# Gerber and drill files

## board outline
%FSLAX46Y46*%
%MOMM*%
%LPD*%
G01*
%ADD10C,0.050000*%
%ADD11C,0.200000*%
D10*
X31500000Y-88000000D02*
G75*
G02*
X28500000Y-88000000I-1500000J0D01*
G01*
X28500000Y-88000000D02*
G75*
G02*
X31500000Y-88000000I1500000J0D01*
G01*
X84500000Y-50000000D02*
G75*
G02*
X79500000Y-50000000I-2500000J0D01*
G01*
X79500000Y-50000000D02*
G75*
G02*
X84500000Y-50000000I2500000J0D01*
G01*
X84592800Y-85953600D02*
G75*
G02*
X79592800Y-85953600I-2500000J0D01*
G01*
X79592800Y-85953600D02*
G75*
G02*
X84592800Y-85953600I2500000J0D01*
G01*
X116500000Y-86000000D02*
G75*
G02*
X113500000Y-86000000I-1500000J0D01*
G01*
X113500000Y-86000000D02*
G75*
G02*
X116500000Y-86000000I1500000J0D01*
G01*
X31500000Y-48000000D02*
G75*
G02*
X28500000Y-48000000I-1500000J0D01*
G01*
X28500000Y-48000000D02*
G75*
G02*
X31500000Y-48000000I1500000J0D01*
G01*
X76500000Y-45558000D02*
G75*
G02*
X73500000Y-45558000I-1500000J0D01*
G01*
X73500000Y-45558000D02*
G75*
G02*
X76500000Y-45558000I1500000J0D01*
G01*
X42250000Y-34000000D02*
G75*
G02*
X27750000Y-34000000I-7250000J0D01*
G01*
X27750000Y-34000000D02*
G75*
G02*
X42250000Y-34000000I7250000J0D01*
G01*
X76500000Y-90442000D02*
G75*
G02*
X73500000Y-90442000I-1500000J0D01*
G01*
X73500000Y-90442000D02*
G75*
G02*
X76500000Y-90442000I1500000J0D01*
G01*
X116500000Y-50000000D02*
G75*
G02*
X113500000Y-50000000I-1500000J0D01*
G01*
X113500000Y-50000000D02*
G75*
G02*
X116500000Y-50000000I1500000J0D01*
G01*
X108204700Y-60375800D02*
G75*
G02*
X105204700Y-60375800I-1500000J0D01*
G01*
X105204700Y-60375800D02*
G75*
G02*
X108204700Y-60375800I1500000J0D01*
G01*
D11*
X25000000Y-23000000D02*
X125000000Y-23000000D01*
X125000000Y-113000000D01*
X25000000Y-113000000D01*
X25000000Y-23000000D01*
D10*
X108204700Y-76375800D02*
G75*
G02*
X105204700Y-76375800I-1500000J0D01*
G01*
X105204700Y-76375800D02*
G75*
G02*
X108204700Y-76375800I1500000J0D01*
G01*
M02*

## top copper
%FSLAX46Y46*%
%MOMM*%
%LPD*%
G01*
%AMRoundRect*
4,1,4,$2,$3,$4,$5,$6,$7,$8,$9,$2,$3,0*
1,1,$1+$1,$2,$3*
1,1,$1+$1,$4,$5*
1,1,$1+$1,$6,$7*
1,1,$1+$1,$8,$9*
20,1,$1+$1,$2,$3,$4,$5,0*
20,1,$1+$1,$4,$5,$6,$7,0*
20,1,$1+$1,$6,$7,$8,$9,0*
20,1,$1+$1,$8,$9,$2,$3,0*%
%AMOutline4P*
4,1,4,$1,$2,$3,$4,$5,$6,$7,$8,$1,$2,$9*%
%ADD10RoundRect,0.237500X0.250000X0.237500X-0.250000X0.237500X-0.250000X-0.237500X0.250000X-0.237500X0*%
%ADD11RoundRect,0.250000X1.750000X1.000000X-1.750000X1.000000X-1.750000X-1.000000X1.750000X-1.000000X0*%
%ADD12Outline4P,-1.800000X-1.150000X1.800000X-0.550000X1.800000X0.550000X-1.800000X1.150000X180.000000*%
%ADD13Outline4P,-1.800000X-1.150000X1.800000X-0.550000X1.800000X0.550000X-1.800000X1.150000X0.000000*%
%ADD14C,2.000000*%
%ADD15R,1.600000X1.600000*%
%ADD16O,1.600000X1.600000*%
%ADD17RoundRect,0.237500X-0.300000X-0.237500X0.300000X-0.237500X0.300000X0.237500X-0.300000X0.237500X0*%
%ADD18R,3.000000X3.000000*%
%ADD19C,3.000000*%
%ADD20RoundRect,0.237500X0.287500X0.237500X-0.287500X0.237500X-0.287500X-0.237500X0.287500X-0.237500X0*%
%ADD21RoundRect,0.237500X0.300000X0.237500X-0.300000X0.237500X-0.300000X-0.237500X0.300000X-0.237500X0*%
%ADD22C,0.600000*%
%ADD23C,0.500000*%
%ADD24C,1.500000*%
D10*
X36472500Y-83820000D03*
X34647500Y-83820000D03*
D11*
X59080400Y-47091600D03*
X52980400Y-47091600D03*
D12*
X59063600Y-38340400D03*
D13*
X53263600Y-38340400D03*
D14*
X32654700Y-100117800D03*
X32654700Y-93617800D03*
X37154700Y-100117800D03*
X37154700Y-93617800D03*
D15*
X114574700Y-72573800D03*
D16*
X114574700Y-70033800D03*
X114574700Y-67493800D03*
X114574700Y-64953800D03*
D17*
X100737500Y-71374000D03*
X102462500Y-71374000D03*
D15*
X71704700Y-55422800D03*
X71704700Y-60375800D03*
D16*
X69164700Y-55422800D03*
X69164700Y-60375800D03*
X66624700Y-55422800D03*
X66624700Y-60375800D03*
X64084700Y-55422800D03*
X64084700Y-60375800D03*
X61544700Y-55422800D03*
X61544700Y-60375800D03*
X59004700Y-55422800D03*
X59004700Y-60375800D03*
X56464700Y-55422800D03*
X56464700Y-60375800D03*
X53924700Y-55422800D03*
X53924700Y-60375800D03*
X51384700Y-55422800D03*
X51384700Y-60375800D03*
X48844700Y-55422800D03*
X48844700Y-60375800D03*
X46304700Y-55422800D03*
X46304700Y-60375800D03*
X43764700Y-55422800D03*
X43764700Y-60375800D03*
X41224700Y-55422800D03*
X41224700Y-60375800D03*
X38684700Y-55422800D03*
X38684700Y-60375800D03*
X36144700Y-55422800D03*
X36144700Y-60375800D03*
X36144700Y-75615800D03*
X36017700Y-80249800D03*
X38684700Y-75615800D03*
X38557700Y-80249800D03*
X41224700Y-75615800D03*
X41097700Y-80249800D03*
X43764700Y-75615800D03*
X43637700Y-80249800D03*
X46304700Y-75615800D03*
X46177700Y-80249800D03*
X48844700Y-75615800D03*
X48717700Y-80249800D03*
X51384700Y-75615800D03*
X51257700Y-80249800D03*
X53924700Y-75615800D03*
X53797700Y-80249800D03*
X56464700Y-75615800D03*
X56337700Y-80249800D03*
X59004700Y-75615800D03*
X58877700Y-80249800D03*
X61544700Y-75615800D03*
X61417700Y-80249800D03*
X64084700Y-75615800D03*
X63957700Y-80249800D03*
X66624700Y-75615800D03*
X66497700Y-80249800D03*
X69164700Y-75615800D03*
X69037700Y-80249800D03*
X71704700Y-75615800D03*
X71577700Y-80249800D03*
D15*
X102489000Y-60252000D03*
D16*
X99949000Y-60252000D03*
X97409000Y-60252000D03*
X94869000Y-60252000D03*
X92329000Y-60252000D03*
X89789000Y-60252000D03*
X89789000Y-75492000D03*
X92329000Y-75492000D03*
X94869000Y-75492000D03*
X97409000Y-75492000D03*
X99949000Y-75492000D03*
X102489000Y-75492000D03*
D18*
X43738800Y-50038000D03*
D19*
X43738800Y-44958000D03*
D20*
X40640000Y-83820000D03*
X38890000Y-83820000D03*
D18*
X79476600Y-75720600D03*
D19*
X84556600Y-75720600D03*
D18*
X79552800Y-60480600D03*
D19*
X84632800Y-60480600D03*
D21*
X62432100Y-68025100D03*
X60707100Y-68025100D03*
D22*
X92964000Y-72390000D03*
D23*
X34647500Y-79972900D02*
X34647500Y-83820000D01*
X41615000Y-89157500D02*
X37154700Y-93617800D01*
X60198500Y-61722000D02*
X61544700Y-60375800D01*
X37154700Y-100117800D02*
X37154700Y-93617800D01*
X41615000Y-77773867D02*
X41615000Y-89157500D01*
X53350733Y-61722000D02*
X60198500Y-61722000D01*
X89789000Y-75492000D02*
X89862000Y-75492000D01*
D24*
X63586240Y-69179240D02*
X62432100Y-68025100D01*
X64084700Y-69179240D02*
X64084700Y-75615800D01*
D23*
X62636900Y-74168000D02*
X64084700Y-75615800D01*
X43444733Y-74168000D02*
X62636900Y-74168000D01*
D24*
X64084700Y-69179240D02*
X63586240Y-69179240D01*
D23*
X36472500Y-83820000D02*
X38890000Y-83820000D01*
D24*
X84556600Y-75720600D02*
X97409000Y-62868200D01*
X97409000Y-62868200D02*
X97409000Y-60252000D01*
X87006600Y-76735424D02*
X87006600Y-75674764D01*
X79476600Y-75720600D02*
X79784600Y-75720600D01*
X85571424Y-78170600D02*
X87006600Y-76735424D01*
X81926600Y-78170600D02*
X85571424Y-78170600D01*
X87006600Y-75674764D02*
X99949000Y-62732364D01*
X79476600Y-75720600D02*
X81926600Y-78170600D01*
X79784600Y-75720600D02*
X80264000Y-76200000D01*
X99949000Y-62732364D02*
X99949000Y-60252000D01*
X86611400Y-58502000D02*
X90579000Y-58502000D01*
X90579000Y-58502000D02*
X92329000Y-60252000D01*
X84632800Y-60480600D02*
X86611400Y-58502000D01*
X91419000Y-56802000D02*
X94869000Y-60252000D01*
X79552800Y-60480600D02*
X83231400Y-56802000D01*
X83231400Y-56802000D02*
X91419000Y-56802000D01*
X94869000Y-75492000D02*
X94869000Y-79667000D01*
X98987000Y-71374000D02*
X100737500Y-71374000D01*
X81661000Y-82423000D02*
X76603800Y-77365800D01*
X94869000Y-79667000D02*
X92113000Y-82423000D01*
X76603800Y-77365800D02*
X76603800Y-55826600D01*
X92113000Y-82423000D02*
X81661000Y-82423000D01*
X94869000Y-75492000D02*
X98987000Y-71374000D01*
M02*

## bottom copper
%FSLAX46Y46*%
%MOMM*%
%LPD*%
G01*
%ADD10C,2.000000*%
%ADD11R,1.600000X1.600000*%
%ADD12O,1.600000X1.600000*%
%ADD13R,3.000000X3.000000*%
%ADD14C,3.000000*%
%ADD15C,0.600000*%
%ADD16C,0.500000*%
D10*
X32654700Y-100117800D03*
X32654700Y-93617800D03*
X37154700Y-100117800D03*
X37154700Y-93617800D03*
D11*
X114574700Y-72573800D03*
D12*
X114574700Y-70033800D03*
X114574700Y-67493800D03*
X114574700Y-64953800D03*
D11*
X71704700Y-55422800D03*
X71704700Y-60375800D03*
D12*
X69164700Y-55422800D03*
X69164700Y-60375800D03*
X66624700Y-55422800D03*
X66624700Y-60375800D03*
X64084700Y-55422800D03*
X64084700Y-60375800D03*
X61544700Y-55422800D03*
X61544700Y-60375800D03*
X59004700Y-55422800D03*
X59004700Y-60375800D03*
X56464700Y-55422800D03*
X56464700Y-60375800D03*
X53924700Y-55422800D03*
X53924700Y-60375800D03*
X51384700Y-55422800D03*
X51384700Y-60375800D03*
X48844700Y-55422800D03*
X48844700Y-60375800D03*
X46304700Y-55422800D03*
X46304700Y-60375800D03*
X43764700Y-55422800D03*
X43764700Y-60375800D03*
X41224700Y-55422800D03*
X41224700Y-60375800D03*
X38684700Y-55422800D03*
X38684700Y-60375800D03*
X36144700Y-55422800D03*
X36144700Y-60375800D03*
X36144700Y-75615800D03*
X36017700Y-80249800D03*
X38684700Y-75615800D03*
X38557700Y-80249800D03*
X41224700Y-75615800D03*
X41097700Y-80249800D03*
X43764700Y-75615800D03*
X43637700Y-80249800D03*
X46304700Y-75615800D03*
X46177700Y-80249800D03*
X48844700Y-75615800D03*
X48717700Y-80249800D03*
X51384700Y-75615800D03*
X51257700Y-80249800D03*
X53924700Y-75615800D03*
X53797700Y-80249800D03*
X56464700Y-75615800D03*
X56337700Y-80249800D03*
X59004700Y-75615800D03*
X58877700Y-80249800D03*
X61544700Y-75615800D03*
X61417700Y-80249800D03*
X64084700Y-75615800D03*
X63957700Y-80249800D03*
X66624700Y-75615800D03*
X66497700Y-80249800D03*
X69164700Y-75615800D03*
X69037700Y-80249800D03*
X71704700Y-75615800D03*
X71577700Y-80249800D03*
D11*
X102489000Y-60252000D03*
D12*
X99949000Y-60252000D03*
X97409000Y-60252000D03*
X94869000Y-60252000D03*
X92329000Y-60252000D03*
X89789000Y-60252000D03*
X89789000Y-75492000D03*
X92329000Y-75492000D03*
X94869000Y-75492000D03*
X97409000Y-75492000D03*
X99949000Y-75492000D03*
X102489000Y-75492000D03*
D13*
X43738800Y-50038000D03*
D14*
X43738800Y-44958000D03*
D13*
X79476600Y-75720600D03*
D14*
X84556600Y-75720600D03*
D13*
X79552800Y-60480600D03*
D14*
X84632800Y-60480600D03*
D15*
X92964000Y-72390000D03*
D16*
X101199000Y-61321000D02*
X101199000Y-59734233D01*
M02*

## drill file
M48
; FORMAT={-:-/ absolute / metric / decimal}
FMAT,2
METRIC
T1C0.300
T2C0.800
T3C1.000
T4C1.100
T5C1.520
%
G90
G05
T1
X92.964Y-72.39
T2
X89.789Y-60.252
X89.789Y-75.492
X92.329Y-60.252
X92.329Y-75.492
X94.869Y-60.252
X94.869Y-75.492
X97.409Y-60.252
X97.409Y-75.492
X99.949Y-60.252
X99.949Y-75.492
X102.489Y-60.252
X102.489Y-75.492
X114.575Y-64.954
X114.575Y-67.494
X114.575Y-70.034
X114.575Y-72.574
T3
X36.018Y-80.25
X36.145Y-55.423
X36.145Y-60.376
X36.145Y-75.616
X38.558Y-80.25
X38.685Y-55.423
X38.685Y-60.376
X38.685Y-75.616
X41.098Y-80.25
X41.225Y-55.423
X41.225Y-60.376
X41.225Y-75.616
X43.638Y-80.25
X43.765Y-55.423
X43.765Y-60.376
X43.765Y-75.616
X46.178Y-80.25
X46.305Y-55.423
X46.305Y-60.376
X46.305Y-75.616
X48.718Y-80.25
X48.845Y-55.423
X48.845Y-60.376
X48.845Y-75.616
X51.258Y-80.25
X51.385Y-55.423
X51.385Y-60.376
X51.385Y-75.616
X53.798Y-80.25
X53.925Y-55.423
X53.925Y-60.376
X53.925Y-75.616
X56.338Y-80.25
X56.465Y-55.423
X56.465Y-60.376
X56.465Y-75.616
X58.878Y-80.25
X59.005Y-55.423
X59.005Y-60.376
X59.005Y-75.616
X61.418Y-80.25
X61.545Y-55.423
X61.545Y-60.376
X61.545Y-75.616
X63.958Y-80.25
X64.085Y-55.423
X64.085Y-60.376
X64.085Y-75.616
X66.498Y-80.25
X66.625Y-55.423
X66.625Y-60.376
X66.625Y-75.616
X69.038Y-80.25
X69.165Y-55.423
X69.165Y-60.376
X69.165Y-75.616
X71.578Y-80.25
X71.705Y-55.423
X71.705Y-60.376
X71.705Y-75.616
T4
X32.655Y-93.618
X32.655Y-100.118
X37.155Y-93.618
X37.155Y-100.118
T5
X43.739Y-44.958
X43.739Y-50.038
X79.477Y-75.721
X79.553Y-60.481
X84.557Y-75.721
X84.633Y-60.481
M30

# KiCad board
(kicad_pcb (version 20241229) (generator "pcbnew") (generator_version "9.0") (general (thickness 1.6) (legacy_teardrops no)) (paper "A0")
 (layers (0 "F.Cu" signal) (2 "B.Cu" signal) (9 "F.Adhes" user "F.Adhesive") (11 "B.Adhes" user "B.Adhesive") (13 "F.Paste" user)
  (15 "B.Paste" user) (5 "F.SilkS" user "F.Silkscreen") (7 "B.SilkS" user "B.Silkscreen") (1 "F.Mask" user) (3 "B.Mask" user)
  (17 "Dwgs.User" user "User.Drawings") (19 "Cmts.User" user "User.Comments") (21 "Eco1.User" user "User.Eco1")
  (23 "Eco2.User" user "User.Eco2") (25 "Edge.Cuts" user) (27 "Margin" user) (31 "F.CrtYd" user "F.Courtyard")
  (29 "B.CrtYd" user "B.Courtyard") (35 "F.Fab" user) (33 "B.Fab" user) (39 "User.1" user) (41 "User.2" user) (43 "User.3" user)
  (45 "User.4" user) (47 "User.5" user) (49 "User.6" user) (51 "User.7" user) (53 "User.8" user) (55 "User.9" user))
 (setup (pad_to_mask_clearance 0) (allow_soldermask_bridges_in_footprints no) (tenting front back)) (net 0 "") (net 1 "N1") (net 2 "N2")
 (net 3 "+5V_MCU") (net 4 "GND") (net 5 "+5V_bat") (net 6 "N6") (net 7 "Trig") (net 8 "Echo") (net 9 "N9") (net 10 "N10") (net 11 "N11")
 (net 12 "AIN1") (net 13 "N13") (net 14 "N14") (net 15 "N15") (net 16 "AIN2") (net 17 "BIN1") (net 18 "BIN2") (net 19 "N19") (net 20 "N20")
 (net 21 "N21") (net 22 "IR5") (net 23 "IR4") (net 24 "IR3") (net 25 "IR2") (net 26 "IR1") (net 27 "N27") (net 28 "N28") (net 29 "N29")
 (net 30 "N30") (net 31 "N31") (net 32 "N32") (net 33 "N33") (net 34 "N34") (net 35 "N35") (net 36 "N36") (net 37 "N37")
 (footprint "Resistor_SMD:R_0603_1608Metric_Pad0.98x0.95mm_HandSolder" (layer "F.Cu") (at 35.56 83.82 180)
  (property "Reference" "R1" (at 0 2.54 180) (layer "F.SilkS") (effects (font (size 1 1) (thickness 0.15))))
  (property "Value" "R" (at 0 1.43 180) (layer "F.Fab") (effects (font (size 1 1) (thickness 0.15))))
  (pad "1" smd roundrect (at -0.9125 0 180) (size 0.975 0.95) (layers "F.Cu" "F.Mask" "F.Paste") (roundrect_rratio 0.25) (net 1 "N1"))
  (pad "2" smd roundrect (at 0.9125 0 180) (size 0.975 0.95) (layers "F.Cu" "F.Mask" "F.Paste") (roundrect_rratio 0.25) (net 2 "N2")))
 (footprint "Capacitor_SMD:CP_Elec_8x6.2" (layer "F.Cu") (at 56.0304 47.0916 180)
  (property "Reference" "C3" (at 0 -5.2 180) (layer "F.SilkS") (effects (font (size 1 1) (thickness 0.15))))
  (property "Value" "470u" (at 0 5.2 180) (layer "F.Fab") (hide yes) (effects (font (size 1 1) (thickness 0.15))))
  (pad "1" smd roundrect (at -3.05 0 180) (size 4 2.5) (layers "F.Cu" "F.Mask" "F.Paste") (roundrect_rratio 0.1) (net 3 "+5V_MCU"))
  (pad "2" smd roundrect (at 3.05 0 180) (size 4 2.5) (layers "F.Cu" "F.Mask" "F.Paste") (roundrect_rratio 0.1) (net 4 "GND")))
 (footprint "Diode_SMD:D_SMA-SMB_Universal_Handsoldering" (layer "F.Cu") (at 56.1636 38.3404 180)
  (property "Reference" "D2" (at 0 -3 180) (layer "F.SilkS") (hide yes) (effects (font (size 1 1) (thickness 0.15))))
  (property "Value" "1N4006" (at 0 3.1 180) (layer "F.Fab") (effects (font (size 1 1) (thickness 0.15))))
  (pad "1" smd trapezoid (at -2.9 0 180) (size 3.6 1.7) (rect_delta 0.6 0) (layers "F.Cu" "F.Mask" "F.Paste") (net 3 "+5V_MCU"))
  (pad "2" smd trapezoid (at 2.9 0) (size 3.6 1.7) (rect_delta 0.6 0) (layers "F.Cu" "F.Mask" "F.Paste") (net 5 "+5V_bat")))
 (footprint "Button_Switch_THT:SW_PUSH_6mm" (layer "F.Cu") (at 32.6547 100.1178 90)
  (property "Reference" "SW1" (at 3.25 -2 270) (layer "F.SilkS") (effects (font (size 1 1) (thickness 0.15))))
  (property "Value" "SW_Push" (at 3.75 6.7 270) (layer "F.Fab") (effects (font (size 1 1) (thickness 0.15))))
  (pad "1" thru_hole circle (at 0 0 180) (size 2 2) (drill 1.1) (layers "*.Cu" "*.Mask") (remove_unused_layers no) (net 4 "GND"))
  (pad "1" thru_hole circle (at 6.5 0 180) (size 2 2) (drill 1.1) (layers "*.Cu" "*.Mask") (remove_unused_layers no) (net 4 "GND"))
  (pad "2" thru_hole circle (at 0 4.5 180) (size 2 2) (drill 1.1) (layers "*.Cu" "*.Mask") (remove_unused_layers no) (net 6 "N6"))
  (pad "2" thru_hole circle (at 6.5 4.5 180) (size 2 2) (drill 1.1) (layers "*.Cu" "*.Mask") (remove_unused_layers no) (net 6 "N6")))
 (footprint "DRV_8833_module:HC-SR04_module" (layer "F.Cu") (at 114.5747 64.4458)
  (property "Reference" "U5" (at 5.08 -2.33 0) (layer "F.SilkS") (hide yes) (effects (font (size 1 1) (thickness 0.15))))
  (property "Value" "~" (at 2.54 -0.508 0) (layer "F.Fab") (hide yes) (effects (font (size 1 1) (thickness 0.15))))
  (pad "1" thru_hole rect (at 0 8.128) (size 1.6 1.6) (drill 0.8) (layers "*.Cu" "*.Mask") (remove_unused_layers no) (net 3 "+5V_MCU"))
  (pad "2" thru_hole oval (at 0 5.588) (size 1.6 1.6) (drill 0.8) (layers "*.Cu" "*.Mask") (remove_unused_layers no) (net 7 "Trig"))
  (pad "3" thru_hole oval (at 0 3.048) (size 1.6 1.6) (drill 0.8) (layers "*.Cu" "*.Mask") (remove_unused_layers no) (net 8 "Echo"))
  (pad "4" thru_hole oval (at 0 0.508) (size 1.6 1.6) (drill 0.8) (layers "*.Cu" "*.Mask") (remove_unused_layers no) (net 4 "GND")))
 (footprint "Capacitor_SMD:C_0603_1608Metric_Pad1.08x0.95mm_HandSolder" (layer "F.Cu") (at 101.6 71.374)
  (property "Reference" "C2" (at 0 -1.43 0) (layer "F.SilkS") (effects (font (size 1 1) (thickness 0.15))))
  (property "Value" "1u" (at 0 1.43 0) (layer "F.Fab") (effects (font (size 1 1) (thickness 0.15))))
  (pad "1" smd roundrect (at -0.8625 0) (size 1.075 0.95) (layers "F.Cu" "F.Mask" "F.Paste") (roundrect_rratio 0.25) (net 5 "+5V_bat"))
  (pad "2" smd roundrect (at 0.8625 0) (size 1.075 0.95) (layers "F.Cu" "F.Mask" "F.Paste") (roundrect_rratio 0.25) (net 4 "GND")))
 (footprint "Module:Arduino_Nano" (layer "F.Cu") (at 71.7047 60.3758 -90)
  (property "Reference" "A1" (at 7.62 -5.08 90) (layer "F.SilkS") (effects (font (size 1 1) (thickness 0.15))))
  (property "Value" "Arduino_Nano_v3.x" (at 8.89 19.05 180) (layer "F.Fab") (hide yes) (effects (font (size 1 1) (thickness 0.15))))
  (pad "1" thru_hole rect (at -4.953 0 270) (size 1.6 1.6) (drill 1) (layers "*.Cu" "*.Mask") (remove_unused_layers no) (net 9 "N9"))
  (pad "1" thru_hole rect (at 0 0 270) (size 1.6 1.6) (drill 1) (layers "*.Cu" "*.Mask") (remove_unused_layers no) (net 9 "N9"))
  (pad "2" thru_hole oval (at -4.953 2.54 270) (size 1.6 1.6) (drill 1) (layers "*.Cu" "*.Mask") (remove_unused_layers no) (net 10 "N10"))
  (pad "2" thru_hole oval (at 0 2.54 270) (size 1.6 1.6) (drill 1) (layers "*.Cu" "*.Mask") (remove_unused_layers no) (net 10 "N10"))
  (pad "3" thru_hole oval (at -4.953 5.08 270) (size 1.6 1.6) (drill 1) (layers "*.Cu" "*.Mask") (remove_unused_layers no) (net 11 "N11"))
  (pad "3" thru_hole oval (at 0 5.08 270) (size 1.6 1.6) (drill 1) (layers "*.Cu" "*.Mask") (remove_unused_layers no) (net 11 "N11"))
  (pad "4" thru_hole oval (at -4.953 7.62 270) (size 1.6 1.6) (drill 1) (layers "*.Cu" "*.Mask") (remove_unused_layers no) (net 4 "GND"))
  (pad "4" thru_hole oval (at 0 7.62 270) (size 1.6 1.6) (drill 1) (layers "*.Cu" "*.Mask") (remove_unused_layers no) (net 4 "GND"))
  (pad "5" thru_hole oval (at -4.953 10.16 270) (size 1.6 1.6) (drill 1) (layers "*.Cu" "*.Mask") (remove_unused_layers no) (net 6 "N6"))
  (pad "5" thru_hole oval (at 0 10.16 270) (size 1.6 1.6) (drill 1) (layers "*.Cu" "*.Mask") (remove_unused_layers no) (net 6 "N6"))
  (pad "6" thru_hole oval (at -4.953 12.7 270) (size 1.6 1.6) (drill 1) (layers "*.Cu" "*.Mask") (remove_unused_layers no) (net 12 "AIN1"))
  (pad "6" thru_hole oval (at 0 12.7 270) (size 1.6 1.6) (drill 1) (layers "*.Cu" "*.Mask") (remove_unused_layers no) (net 12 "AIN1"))
  (pad "7" thru_hole oval (at -4.953 15.24 270) (size 1.6 1.6) (drill 1) (layers "*.Cu" "*.Mask") (remove_unused_layers no) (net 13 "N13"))
  (pad "7" thru_hole oval (at 0 15.24 270) (size 1.6 1.6) (drill 1) (layers "*.Cu" "*.Mask") (remove_unused_layers no) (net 13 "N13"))
  (pad "8" thru_hole oval (at -4.953 17.78 270) (size 1.6 1.6) (drill 1) (layers "*.Cu" "*.Mask") (remove_unused_layers no) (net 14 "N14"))
  (pad "8" thru_hole oval (at 0 17.78 270) (size 1.6 1.6) (drill 1) (layers "*.Cu" "*.Mask") (remove_unused_layers no) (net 14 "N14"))
  (pad "9" thru_hole oval (at -4.953 20.32 270) (size 1.6 1.6) (drill 1) (layers "*.Cu" "*.Mask") (remove_unused_layers no) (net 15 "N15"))
  (pad "9" thru_hole oval (at 0 20.32 270) (size 1.6 1.6) (drill 1) (layers "*.Cu" "*.Mask") (remove_unused_layers no) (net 15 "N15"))
  (pad "10" thru_hole oval (at -4.953 22.86 270) (size 1.6 1.6) (drill 1) (layers "*.Cu" "*.Mask") (remove_unused_layers no) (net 7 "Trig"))
  (pad "10" thru_hole oval (at 0 22.86 270) (size 1.6 1.6) (drill 1) (layers "*.Cu" "*.Mask") (remove_unused_layers no) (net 7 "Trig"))
  (pad "11" thru_hole oval (at -4.953 25.4 270) (size 1.6 1.6) (drill 1) (layers "*.Cu" "*.Mask") (remove_unused_layers no) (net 8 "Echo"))
  (pad "11" thru_hole oval (at 0 25.4 270) (size 1.6 1.6) (drill 1) (layers "*.Cu" "*.Mask") (remove_unused_layers no) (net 8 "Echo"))
  (pad "12" thru_hole oval (at -4.953 27.94 270) (size 1.6 1.6) (drill 1) (layers "*.Cu" "*.Mask") (remove_unused_layers no) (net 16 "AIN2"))
  (pad "12" thru_hole oval (at 0 27.94 270) (size 1.6 1.6) (drill 1) (layers "*.Cu" "*.Mask") (remove_unused_layers no) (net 16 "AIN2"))
  (pad "13" thru_hole oval (at -4.953 30.48 270) (size 1.6 1.6) (drill 1) (layers "*.Cu" "*.Mask") (remove_unused_layers no) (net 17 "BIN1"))
  (pad "13" thru_hole oval (at 0 30.48 270) (size 1.6 1.6) (drill 1) (layers "*.Cu" "*.Mask") (remove_unused_layers no) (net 17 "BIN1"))
  (pad "14" thru_hole oval (at -4.953 33.02 270) (size 1.6 1.6) (drill 1) (layers "*.Cu" "*.Mask") (remove_unused_layers no) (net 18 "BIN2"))
  (pad "14" thru_hole oval (at 0 33.02 270) (size 1.6 1.6) (drill 1) (layers "*.Cu" "*.Mask") (remove_unused_layers no) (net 18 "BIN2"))
  (pad "15" thru_hole oval (at -4.953 35.56 270) (size 1.6 1.6) (drill 1) (layers "*.Cu" "*.Mask") (remove_unused_layers no) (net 2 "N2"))
  (pad "15" thru_hole oval (at 0 35.56 270) (size 1.6 1.6) (drill 1) (layers "*.Cu" "*.Mask") (remove_unused_layers no) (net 2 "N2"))
  (pad "16" thru_hole oval (at 15.24 35.56 270) (size 1.6 1.6) (drill 1) (layers "*.Cu" "*.Mask") (remove_unused_layers no) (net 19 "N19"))
  (pad "16" thru_hole oval (at 19.874 35.687 270) (size 1.6 1.6) (drill 1) (layers "*.Cu" "*.Mask") (remove_unused_layers no) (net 19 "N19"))
  (pad "17" thru_hole oval (at 15.24 33.02 270) (size 1.6 1.6) (drill 1) (layers "*.Cu" "*.Mask") (remove_unused_layers no) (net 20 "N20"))
  (pad "17" thru_hole oval (at 19.874 33.147 270) (size 1.6 1.6) (drill 1) (layers "*.Cu" "*.Mask") (remove_unused_layers no) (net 20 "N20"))
  (pad "18" thru_hole oval (at 15.24 30.48 270) (size 1.6 1.6) (drill 1) (layers "*.Cu" "*.Mask") (remove_unused_layers no) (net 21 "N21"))
  (pad "18" thru_hole oval (at 19.874 30.607 270) (size 1.6 1.6) (drill 1) (layers "*.Cu" "*.Mask") (remove_unused_layers no) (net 21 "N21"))
  (pad "19" thru_hole oval (at 15.24 27.94 270) (size 1.6 1.6) (drill 1) (layers "*.Cu" "*.Mask") (remove_unused_layers no) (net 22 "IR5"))
  (pad "19" thru_hole oval (at 19.874 28.067 270) (size 1.6 1.6) (drill 1) (layers "*.Cu" "*.Mask") (remove_unused_layers no) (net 22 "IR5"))
  (pad "20" thru_hole oval (at 15.24 25.4 270) (size 1.6 1.6) (drill 1) (layers "*.Cu" "*.Mask") (remove_unused_layers no) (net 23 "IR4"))
  (pad "20" thru_hole oval (at 19.874 25.527 270) (size 1.6 1.6) (drill 1) (layers "*.Cu" "*.Mask") (remove_unused_layers no) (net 23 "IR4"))
  (pad "21" thru_hole oval (at 15.24 22.86 270) (size 1.6 1.6) (drill 1) (layers "*.Cu" "*.Mask") (remove_unused_layers no) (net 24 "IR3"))
  (pad "21" thru_hole oval (at 19.874 22.987 270) (size 1.6 1.6) (drill 1) (layers "*.Cu" "*.Mask") (remove_unused_layers no) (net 24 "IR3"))
  (pad "22" thru_hole oval (at 15.24 20.32 270) (size 1.6 1.6) (drill 1) (layers "*.Cu" "*.Mask") (remove_unused_layers no) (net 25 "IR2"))
  (pad "22" thru_hole oval (at 19.874 20.447 270) (size 1.6 1.6) (drill 1) (layers "*.Cu" "*.Mask") (remove_unused_layers no) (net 25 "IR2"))
  (pad "23" thru_hole oval (at 15.24 17.78 270) (size 1.6 1.6) (drill 1) (layers "*.Cu" "*.Mask") (remove_unused_layers no) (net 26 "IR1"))
  (pad "23" thru_hole oval (at 19.874 17.907 270) (size 1.6 1.6) (drill 1) (layers "*.Cu" "*.Mask") (remove_unused_layers no) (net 26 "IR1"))
  (pad "24" thru_hole oval (at 15.24 15.24 270) (size 1.6 1.6) (drill 1) (layers "*.Cu" "*.Mask") (remove_unused_layers no) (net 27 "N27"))
  (pad "24" thru_hole oval (at 19.874 15.367 270) (size 1.6 1.6) (drill 1) (layers "*.Cu" "*.Mask") (remove_unused_layers no) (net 27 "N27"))
  (pad "25" thru_hole oval (at 15.24 12.7 270) (size 1.6 1.6) (drill 1) (layers "*.Cu" "*.Mask") (remove_unused_layers no) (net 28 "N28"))
  (pad "25" thru_hole oval (at 19.874 12.827 270) (size 1.6 1.6) (drill 1) (layers "*.Cu" "*.Mask") (remove_unused_layers no) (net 28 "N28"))
  (pad "26" thru_hole oval (at 15.24 10.16 270) (size 1.6 1.6) (drill 1) (layers "*.Cu" "*.Mask") (remove_unused_layers no) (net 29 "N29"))
  (pad "26" thru_hole oval (at 19.874 10.287 270) (size 1.6 1.6) (drill 1) (layers "*.Cu" "*.Mask") (remove_unused_layers no) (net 29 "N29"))
  (pad "27" thru_hole oval (at 15.24 7.62 270) (size 1.6 1.6) (drill 1) (layers "*.Cu" "*.Mask") (remove_unused_layers no) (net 3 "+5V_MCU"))
  (pad "27" thru_hole oval (at 19.874 7.747 270) (size 1.6 1.6) (drill 1) (layers "*.Cu" "*.Mask") (remove_unused_layers no)
   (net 3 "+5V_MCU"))
  (pad "28" thru_hole oval (at 15.24 5.08 270) (size 1.6 1.6) (drill 1) (layers "*.Cu" "*.Mask") (remove_unused_layers no) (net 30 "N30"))
  (pad "28" thru_hole oval (at 19.874 5.207 270) (size 1.6 1.6) (drill 1) (layers "*.Cu" "*.Mask") (remove_unused_layers no) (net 30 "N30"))
  (pad "29" thru_hole oval (at 15.24 2.54 270) (size 1.6 1.6) (drill 1) (layers "*.Cu" "*.Mask") (remove_unused_layers no) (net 4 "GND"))
  (pad "29" thru_hole oval (at 19.874 2.667 270) (size 1.6 1.6) (drill 1) (layers "*.Cu" "*.Mask") (remove_unused_layers no) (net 4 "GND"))
  (pad "30" thru_hole oval (at 15.24 0 270) (size 1.6 1.6) (drill 1) (layers "*.Cu" "*.Mask") (remove_unused_layers no) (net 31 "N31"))
  (pad "30" thru_hole oval (at 19.874 0.127 270) (size 1.6 1.6) (drill 1) (layers "*.Cu" "*.Mask") (remove_unused_layers no) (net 31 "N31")))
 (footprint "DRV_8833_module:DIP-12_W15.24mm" (layer "F.Cu") (at 102.489 60.252 -90)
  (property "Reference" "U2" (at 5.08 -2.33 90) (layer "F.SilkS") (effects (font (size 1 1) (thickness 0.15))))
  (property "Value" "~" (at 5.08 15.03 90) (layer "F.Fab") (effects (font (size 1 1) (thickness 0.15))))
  (pad "1" thru_hole rect (at 0 0 270) (size 1.6 1.6) (drill 0.8) (layers "*.Cu" "*.Mask") (remove_unused_layers no) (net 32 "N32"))
  (pad "2" thru_hole oval (at 0 2.54 270) (size 1.6 1.6) (drill 0.8) (layers "*.Cu" "*.Mask") (remove_unused_layers no) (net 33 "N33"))
  (pad "3" thru_hole oval (at 0 5.08 270) (size 1.6 1.6) (drill 0.8) (layers "*.Cu" "*.Mask") (remove_unused_layers no) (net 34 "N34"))
  (pad "4" thru_hole oval (at 0 7.62 270) (size 1.6 1.6) (drill 0.8) (layers "*.Cu" "*.Mask") (remove_unused_layers no) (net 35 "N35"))
  (pad "5" thru_hole oval (at 0 10.16 270) (size 1.6 1.6) (drill 0.8) (layers "*.Cu" "*.Mask") (remove_unused_layers no) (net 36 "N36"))
  (pad "6" thru_hole oval (at 0 12.7 270) (size 1.6 1.6) (drill 0.8) (layers "*.Cu" "*.Mask") (remove_unused_layers no) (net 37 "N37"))
  (pad "7" thru_hole oval (at 15.24 12.7 270) (size 1.6 1.6) (drill 0.8) (layers "*.Cu" "*.Mask") (remove_unused_layers no) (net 12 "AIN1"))
  (pad "8" thru_hole oval (at 15.24 10.16 270) (size 1.6 1.6) (drill 0.8) (layers "*.Cu" "*.Mask") (remove_unused_layers no) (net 16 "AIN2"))
  (pad "9" thru_hole oval (at 15.24 7.62 270) (size 1.6 1.6) (drill 0.8) (layers "*.Cu" "*.Mask") (remove_unused_layers no)
   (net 5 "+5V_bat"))
  (pad "10" thru_hole oval (at 15.24 5.08 270) (size 1.6 1.6) (drill 0.8) (layers "*.Cu" "*.Mask") (remove_unused_layers no) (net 4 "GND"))
  (pad "11" thru_hole oval (at 15.24 2.54 270) (size 1.6 1.6) (drill 0.8) (layers "*.Cu" "*.Mask") (remove_unused_layers no) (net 17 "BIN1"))
  (pad "12" thru_hole oval (at 15.24 0 270) (size 1.6 1.6) (drill 0.8) (layers "*.Cu" "*.Mask") (remove_unused_layers no) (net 18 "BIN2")))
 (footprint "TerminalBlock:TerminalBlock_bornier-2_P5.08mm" (layer "F.Cu") (at 43.7388 50.038 90)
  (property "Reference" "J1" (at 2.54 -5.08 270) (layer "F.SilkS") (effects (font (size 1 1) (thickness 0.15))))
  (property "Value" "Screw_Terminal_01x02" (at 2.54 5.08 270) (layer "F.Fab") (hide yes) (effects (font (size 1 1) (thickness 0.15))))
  (pad "1" thru_hole rect (at 0 0 90) (size 3 3) (drill 1.52) (layers "*.Cu" "*.Mask") (remove_unused_layers no) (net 4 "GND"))
  (pad "2" thru_hole circle (at 5.08 0 90) (size 3 3) (drill 1.52) (layers "*.Cu" "*.Mask") (remove_unused_layers no) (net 5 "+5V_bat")))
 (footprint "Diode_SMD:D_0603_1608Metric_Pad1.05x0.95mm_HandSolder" (layer "F.Cu") (at 39.765 83.82 180)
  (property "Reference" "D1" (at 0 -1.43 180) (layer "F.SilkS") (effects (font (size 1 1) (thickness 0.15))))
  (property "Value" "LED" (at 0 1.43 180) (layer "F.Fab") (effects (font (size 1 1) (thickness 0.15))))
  (pad "1" smd roundrect (at -0.875 0 180) (size 1.05 0.95) (layers "F.Cu" "F.Mask" "F.Paste") (roundrect_rratio 0.25) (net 4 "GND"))
  (pad "2" smd roundrect (at 0.875 0 180) (size 1.05 0.95) (layers "F.Cu" "F.Mask" "F.Paste") (roundrect_rratio 0.25) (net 1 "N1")))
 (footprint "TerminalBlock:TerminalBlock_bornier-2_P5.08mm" (layer "F.Cu") (at 79.4766 75.7206)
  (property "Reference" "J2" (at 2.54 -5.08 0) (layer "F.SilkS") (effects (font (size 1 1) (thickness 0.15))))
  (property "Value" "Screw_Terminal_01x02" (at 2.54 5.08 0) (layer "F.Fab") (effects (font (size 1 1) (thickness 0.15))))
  (pad "1" thru_hole rect (at 0 0) (size 3 3) (drill 1.52) (layers "*.Cu" "*.Mask") (remove_unused_layers no) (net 33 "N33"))
  (pad "2" thru_hole circle (at 5.08 0) (size 3 3) (drill 1.52) (layers "*.Cu" "*.Mask") (remove_unused_layers no) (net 34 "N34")))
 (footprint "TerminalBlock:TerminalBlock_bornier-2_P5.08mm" (layer "F.Cu") (at 79.5528 60.4806)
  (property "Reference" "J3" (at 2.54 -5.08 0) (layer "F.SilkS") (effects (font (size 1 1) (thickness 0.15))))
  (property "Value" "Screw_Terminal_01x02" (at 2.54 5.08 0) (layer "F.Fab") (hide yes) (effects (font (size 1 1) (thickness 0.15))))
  (pad "1" thru_hole rect (at 0 0) (size 3 3) (drill 1.52) (layers "*.Cu" "*.Mask") (remove_unused_layers no) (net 35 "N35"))
  (pad "2" thru_hole circle (at 5.08 0) (size 3 3) (drill 1.52) (layers "*.Cu" "*.Mask") (remove_unused_layers no) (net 36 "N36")))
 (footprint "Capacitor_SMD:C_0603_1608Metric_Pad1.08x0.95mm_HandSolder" (layer "F.Cu") (at 61.5696 68.0251 180)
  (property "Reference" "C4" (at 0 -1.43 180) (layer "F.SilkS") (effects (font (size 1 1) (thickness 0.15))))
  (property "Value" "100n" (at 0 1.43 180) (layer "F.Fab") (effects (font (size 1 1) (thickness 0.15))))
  (pad "1" smd roundrect (at -0.8625 0 180) (size 1.075 0.95) (layers "F.Cu" "F.Mask" "F.Paste") (roundrect_rratio 0.25) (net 3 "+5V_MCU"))
  (pad "2" smd roundrect (at 0.8625 0 180) (size 1.075 0.95) (layers "F.Cu" "F.Mask" "F.Paste") (roundrect_rratio 0.25) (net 4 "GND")))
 (gr_circle (center 30 88) (end 31.5 88) (stroke (width 0.05) (type default)) (fill no) (layer "Edge.Cuts"))
 (gr_circle (center 82 50) (end 84.5 50) (stroke (width 0.05) (type solid)) (fill no) (layer "Edge.Cuts"))
 (gr_circle (center 82.0928 85.9536) (end 84.5928 85.9536) (stroke (width 0.05) (type solid)) (fill no) (layer "Edge.Cuts"))
 (gr_circle (center 115 86) (end 116.5 86) (stroke (width 0.05) (type default)) (fill no) (layer "Edge.Cuts"))
 (gr_circle (center 30 48) (end 31.5 48) (stroke (width 0.05) (type default)) (fill no) (layer "Edge.Cuts"))
 (gr_circle (center 75 45.558) (end 76.5 45.558) (stroke (width 0.05) (type default)) (fill no) (layer "Edge.Cuts"))
 (gr_circle (center 35 34) (end 42.25 34) (stroke (width 0.05) (type solid)) (fill no) (layer "Edge.Cuts"))
 (gr_circle (center 75 90.442) (end 76.5 90.442) (stroke (width 0.05) (type default)) (fill no) (layer "Edge.Cuts"))
 (gr_circle (center 115 50) (end 116.5 50) (stroke (width 0.05) (type default)) (fill no) (layer "Edge.Cuts"))
 (gr_circle (center 106.7047 60.3758) (end 108.2047 60.3758) (stroke (width 0.05) (type default)) (fill no) (layer "Edge.Cuts"))
 (gr_rect (start 25 23) (end 125 113) (stroke (width 0.2) (type default)) (fill no) (layer "Edge.Cuts"))
 (gr_circle (center 106.7047 76.3758) (end 108.2047 76.3758) (stroke (width 0.05) (type default)) (fill no) (layer "Edge.Cuts"))
 (segment (start 34.6475 79.9729) (end 34.6475 83.82) (width 0.5) (layer "F.Cu") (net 2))
 (segment (start 41.615 89.1575) (end 37.1547 93.6178) (width 0.5) (layer "F.Cu") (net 6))
 (segment (start 60.1985 61.722) (end 61.5447 60.3758) (width 0.5) (layer "F.Cu") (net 6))
 (segment (start 37.1547 100.1178) (end 37.1547 93.6178) (width 0.5) (layer "F.Cu") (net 6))
 (segment (start 41.615 77.773867) (end 41.615 89.1575) (width 0.5) (layer "F.Cu") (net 6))
 (segment (start 53.350733 61.722) (end 60.1985 61.722) (width 0.5) (layer "F.Cu") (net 6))
 (segment (start 89.789 75.492) (end 89.862 75.492) (width 0.5) (layer "F.Cu") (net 12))
 (via (at 92.964 72.39) (size 0.6) (drill 0.3) (layers "F.Cu" "B.Cu") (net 12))
 (segment (start 63.58624 69.17924) (end 62.4321 68.0251) (width 1.5) (layer "F.Cu") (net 3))
 (segment (start 64.0847 69.17924) (end 64.0847 75.6158) (width 1.5) (layer "F.Cu") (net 3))
 (segment (start 62.6369 74.168) (end 64.0847 75.6158) (width 0.5) (layer "F.Cu") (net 3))
 (segment (start 43.444733 74.168) (end 62.6369 74.168) (width 0.5) (layer "F.Cu") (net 3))
 (segment (start 64.0847 69.17924) (end 63.58624 69.17924) (width 1.5) (layer "F.Cu") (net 3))
 (segment (start 101.199 61.321) (end 101.199 59.734233) (width 0.5) (layer "B.Cu") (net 8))
 (segment (start 36.4725 83.82) (end 38.89 83.82) (width 0.5) (layer "F.Cu") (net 1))
 (segment (start 84.5566 75.7206) (end 97.409 62.8682) (width 1.5) (layer "F.Cu") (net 34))
 (segment (start 97.409 62.8682) (end 97.409 60.252) (width 1.5) (layer "F.Cu") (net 34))
 (segment (start 87.0066 76.735424) (end 87.0066 75.674764) (width 1.5) (layer "F.Cu") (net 33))
 (segment (start 79.4766 75.7206) (end 79.7846 75.7206) (width 1.5) (layer "F.Cu") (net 33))
 (segment (start 85.571424 78.1706) (end 87.0066 76.735424) (width 1.5) (layer "F.Cu") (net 33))
 (segment (start 81.9266 78.1706) (end 85.571424 78.1706) (width 1.5) (layer "F.Cu") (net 33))
 (segment (start 87.0066 75.674764) (end 99.949 62.732364) (width 1.5) (layer "F.Cu") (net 33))
 (segment (start 79.4766 75.7206) (end 81.9266 78.1706) (width 1.5) (layer "F.Cu") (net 33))
 (segment (start 79.7846 75.7206) (end 80.264 76.2) (width 1.5) (layer "F.Cu") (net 33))
 (segment (start 99.949 62.732364) (end 99.949 60.252) (width 1.5) (layer "F.Cu") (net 33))
 (segment (start 86.6114 58.502) (end 90.579 58.502) (width 1.5) (layer "F.Cu") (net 36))
 (segment (start 90.579 58.502) (end 92.329 60.252) (width 1.5) (layer "F.Cu") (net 36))
 (segment (start 84.6328 60.4806) (end 86.6114 58.502) (width 1.5) (layer "F.Cu") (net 36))
 (segment (start 91.419 56.802) (end 94.869 60.252) (width 1.5) (layer "F.Cu") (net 35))
 (segment (start 79.5528 60.4806) (end 83.2314 56.802) (width 1.5) (layer "F.Cu") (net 35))
 (segment (start 83.2314 56.802) (end 91.419 56.802) (width 1.5) (layer "F.Cu") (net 35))
 (segment (start 94.869 75.492) (end 94.869 79.667) (width 1.5) (layer "F.Cu") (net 5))
 (segment (start 98.987 71.374) (end 100.7375 71.374) (width 1.5) (layer "F.Cu") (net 5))
 (segment (start 81.661 82.423) (end 76.6038 77.3658) (width 1.5) (layer "F.Cu") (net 5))
 (segment (start 94.869 79.667) (end 92.113 82.423) (width 1.5) (layer "F.Cu") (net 5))
 (segment (start 76.6038 77.3658) (end 76.6038 55.8266) (width 1.5) (layer "F.Cu") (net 5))
 (segment (start 92.113 82.423) (end 81.661 82.423) (width 1.5) (layer "F.Cu") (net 5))
 (segment (start 94.869 75.492) (end 98.987 71.374) (width 1.5) (layer "F.Cu") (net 5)))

